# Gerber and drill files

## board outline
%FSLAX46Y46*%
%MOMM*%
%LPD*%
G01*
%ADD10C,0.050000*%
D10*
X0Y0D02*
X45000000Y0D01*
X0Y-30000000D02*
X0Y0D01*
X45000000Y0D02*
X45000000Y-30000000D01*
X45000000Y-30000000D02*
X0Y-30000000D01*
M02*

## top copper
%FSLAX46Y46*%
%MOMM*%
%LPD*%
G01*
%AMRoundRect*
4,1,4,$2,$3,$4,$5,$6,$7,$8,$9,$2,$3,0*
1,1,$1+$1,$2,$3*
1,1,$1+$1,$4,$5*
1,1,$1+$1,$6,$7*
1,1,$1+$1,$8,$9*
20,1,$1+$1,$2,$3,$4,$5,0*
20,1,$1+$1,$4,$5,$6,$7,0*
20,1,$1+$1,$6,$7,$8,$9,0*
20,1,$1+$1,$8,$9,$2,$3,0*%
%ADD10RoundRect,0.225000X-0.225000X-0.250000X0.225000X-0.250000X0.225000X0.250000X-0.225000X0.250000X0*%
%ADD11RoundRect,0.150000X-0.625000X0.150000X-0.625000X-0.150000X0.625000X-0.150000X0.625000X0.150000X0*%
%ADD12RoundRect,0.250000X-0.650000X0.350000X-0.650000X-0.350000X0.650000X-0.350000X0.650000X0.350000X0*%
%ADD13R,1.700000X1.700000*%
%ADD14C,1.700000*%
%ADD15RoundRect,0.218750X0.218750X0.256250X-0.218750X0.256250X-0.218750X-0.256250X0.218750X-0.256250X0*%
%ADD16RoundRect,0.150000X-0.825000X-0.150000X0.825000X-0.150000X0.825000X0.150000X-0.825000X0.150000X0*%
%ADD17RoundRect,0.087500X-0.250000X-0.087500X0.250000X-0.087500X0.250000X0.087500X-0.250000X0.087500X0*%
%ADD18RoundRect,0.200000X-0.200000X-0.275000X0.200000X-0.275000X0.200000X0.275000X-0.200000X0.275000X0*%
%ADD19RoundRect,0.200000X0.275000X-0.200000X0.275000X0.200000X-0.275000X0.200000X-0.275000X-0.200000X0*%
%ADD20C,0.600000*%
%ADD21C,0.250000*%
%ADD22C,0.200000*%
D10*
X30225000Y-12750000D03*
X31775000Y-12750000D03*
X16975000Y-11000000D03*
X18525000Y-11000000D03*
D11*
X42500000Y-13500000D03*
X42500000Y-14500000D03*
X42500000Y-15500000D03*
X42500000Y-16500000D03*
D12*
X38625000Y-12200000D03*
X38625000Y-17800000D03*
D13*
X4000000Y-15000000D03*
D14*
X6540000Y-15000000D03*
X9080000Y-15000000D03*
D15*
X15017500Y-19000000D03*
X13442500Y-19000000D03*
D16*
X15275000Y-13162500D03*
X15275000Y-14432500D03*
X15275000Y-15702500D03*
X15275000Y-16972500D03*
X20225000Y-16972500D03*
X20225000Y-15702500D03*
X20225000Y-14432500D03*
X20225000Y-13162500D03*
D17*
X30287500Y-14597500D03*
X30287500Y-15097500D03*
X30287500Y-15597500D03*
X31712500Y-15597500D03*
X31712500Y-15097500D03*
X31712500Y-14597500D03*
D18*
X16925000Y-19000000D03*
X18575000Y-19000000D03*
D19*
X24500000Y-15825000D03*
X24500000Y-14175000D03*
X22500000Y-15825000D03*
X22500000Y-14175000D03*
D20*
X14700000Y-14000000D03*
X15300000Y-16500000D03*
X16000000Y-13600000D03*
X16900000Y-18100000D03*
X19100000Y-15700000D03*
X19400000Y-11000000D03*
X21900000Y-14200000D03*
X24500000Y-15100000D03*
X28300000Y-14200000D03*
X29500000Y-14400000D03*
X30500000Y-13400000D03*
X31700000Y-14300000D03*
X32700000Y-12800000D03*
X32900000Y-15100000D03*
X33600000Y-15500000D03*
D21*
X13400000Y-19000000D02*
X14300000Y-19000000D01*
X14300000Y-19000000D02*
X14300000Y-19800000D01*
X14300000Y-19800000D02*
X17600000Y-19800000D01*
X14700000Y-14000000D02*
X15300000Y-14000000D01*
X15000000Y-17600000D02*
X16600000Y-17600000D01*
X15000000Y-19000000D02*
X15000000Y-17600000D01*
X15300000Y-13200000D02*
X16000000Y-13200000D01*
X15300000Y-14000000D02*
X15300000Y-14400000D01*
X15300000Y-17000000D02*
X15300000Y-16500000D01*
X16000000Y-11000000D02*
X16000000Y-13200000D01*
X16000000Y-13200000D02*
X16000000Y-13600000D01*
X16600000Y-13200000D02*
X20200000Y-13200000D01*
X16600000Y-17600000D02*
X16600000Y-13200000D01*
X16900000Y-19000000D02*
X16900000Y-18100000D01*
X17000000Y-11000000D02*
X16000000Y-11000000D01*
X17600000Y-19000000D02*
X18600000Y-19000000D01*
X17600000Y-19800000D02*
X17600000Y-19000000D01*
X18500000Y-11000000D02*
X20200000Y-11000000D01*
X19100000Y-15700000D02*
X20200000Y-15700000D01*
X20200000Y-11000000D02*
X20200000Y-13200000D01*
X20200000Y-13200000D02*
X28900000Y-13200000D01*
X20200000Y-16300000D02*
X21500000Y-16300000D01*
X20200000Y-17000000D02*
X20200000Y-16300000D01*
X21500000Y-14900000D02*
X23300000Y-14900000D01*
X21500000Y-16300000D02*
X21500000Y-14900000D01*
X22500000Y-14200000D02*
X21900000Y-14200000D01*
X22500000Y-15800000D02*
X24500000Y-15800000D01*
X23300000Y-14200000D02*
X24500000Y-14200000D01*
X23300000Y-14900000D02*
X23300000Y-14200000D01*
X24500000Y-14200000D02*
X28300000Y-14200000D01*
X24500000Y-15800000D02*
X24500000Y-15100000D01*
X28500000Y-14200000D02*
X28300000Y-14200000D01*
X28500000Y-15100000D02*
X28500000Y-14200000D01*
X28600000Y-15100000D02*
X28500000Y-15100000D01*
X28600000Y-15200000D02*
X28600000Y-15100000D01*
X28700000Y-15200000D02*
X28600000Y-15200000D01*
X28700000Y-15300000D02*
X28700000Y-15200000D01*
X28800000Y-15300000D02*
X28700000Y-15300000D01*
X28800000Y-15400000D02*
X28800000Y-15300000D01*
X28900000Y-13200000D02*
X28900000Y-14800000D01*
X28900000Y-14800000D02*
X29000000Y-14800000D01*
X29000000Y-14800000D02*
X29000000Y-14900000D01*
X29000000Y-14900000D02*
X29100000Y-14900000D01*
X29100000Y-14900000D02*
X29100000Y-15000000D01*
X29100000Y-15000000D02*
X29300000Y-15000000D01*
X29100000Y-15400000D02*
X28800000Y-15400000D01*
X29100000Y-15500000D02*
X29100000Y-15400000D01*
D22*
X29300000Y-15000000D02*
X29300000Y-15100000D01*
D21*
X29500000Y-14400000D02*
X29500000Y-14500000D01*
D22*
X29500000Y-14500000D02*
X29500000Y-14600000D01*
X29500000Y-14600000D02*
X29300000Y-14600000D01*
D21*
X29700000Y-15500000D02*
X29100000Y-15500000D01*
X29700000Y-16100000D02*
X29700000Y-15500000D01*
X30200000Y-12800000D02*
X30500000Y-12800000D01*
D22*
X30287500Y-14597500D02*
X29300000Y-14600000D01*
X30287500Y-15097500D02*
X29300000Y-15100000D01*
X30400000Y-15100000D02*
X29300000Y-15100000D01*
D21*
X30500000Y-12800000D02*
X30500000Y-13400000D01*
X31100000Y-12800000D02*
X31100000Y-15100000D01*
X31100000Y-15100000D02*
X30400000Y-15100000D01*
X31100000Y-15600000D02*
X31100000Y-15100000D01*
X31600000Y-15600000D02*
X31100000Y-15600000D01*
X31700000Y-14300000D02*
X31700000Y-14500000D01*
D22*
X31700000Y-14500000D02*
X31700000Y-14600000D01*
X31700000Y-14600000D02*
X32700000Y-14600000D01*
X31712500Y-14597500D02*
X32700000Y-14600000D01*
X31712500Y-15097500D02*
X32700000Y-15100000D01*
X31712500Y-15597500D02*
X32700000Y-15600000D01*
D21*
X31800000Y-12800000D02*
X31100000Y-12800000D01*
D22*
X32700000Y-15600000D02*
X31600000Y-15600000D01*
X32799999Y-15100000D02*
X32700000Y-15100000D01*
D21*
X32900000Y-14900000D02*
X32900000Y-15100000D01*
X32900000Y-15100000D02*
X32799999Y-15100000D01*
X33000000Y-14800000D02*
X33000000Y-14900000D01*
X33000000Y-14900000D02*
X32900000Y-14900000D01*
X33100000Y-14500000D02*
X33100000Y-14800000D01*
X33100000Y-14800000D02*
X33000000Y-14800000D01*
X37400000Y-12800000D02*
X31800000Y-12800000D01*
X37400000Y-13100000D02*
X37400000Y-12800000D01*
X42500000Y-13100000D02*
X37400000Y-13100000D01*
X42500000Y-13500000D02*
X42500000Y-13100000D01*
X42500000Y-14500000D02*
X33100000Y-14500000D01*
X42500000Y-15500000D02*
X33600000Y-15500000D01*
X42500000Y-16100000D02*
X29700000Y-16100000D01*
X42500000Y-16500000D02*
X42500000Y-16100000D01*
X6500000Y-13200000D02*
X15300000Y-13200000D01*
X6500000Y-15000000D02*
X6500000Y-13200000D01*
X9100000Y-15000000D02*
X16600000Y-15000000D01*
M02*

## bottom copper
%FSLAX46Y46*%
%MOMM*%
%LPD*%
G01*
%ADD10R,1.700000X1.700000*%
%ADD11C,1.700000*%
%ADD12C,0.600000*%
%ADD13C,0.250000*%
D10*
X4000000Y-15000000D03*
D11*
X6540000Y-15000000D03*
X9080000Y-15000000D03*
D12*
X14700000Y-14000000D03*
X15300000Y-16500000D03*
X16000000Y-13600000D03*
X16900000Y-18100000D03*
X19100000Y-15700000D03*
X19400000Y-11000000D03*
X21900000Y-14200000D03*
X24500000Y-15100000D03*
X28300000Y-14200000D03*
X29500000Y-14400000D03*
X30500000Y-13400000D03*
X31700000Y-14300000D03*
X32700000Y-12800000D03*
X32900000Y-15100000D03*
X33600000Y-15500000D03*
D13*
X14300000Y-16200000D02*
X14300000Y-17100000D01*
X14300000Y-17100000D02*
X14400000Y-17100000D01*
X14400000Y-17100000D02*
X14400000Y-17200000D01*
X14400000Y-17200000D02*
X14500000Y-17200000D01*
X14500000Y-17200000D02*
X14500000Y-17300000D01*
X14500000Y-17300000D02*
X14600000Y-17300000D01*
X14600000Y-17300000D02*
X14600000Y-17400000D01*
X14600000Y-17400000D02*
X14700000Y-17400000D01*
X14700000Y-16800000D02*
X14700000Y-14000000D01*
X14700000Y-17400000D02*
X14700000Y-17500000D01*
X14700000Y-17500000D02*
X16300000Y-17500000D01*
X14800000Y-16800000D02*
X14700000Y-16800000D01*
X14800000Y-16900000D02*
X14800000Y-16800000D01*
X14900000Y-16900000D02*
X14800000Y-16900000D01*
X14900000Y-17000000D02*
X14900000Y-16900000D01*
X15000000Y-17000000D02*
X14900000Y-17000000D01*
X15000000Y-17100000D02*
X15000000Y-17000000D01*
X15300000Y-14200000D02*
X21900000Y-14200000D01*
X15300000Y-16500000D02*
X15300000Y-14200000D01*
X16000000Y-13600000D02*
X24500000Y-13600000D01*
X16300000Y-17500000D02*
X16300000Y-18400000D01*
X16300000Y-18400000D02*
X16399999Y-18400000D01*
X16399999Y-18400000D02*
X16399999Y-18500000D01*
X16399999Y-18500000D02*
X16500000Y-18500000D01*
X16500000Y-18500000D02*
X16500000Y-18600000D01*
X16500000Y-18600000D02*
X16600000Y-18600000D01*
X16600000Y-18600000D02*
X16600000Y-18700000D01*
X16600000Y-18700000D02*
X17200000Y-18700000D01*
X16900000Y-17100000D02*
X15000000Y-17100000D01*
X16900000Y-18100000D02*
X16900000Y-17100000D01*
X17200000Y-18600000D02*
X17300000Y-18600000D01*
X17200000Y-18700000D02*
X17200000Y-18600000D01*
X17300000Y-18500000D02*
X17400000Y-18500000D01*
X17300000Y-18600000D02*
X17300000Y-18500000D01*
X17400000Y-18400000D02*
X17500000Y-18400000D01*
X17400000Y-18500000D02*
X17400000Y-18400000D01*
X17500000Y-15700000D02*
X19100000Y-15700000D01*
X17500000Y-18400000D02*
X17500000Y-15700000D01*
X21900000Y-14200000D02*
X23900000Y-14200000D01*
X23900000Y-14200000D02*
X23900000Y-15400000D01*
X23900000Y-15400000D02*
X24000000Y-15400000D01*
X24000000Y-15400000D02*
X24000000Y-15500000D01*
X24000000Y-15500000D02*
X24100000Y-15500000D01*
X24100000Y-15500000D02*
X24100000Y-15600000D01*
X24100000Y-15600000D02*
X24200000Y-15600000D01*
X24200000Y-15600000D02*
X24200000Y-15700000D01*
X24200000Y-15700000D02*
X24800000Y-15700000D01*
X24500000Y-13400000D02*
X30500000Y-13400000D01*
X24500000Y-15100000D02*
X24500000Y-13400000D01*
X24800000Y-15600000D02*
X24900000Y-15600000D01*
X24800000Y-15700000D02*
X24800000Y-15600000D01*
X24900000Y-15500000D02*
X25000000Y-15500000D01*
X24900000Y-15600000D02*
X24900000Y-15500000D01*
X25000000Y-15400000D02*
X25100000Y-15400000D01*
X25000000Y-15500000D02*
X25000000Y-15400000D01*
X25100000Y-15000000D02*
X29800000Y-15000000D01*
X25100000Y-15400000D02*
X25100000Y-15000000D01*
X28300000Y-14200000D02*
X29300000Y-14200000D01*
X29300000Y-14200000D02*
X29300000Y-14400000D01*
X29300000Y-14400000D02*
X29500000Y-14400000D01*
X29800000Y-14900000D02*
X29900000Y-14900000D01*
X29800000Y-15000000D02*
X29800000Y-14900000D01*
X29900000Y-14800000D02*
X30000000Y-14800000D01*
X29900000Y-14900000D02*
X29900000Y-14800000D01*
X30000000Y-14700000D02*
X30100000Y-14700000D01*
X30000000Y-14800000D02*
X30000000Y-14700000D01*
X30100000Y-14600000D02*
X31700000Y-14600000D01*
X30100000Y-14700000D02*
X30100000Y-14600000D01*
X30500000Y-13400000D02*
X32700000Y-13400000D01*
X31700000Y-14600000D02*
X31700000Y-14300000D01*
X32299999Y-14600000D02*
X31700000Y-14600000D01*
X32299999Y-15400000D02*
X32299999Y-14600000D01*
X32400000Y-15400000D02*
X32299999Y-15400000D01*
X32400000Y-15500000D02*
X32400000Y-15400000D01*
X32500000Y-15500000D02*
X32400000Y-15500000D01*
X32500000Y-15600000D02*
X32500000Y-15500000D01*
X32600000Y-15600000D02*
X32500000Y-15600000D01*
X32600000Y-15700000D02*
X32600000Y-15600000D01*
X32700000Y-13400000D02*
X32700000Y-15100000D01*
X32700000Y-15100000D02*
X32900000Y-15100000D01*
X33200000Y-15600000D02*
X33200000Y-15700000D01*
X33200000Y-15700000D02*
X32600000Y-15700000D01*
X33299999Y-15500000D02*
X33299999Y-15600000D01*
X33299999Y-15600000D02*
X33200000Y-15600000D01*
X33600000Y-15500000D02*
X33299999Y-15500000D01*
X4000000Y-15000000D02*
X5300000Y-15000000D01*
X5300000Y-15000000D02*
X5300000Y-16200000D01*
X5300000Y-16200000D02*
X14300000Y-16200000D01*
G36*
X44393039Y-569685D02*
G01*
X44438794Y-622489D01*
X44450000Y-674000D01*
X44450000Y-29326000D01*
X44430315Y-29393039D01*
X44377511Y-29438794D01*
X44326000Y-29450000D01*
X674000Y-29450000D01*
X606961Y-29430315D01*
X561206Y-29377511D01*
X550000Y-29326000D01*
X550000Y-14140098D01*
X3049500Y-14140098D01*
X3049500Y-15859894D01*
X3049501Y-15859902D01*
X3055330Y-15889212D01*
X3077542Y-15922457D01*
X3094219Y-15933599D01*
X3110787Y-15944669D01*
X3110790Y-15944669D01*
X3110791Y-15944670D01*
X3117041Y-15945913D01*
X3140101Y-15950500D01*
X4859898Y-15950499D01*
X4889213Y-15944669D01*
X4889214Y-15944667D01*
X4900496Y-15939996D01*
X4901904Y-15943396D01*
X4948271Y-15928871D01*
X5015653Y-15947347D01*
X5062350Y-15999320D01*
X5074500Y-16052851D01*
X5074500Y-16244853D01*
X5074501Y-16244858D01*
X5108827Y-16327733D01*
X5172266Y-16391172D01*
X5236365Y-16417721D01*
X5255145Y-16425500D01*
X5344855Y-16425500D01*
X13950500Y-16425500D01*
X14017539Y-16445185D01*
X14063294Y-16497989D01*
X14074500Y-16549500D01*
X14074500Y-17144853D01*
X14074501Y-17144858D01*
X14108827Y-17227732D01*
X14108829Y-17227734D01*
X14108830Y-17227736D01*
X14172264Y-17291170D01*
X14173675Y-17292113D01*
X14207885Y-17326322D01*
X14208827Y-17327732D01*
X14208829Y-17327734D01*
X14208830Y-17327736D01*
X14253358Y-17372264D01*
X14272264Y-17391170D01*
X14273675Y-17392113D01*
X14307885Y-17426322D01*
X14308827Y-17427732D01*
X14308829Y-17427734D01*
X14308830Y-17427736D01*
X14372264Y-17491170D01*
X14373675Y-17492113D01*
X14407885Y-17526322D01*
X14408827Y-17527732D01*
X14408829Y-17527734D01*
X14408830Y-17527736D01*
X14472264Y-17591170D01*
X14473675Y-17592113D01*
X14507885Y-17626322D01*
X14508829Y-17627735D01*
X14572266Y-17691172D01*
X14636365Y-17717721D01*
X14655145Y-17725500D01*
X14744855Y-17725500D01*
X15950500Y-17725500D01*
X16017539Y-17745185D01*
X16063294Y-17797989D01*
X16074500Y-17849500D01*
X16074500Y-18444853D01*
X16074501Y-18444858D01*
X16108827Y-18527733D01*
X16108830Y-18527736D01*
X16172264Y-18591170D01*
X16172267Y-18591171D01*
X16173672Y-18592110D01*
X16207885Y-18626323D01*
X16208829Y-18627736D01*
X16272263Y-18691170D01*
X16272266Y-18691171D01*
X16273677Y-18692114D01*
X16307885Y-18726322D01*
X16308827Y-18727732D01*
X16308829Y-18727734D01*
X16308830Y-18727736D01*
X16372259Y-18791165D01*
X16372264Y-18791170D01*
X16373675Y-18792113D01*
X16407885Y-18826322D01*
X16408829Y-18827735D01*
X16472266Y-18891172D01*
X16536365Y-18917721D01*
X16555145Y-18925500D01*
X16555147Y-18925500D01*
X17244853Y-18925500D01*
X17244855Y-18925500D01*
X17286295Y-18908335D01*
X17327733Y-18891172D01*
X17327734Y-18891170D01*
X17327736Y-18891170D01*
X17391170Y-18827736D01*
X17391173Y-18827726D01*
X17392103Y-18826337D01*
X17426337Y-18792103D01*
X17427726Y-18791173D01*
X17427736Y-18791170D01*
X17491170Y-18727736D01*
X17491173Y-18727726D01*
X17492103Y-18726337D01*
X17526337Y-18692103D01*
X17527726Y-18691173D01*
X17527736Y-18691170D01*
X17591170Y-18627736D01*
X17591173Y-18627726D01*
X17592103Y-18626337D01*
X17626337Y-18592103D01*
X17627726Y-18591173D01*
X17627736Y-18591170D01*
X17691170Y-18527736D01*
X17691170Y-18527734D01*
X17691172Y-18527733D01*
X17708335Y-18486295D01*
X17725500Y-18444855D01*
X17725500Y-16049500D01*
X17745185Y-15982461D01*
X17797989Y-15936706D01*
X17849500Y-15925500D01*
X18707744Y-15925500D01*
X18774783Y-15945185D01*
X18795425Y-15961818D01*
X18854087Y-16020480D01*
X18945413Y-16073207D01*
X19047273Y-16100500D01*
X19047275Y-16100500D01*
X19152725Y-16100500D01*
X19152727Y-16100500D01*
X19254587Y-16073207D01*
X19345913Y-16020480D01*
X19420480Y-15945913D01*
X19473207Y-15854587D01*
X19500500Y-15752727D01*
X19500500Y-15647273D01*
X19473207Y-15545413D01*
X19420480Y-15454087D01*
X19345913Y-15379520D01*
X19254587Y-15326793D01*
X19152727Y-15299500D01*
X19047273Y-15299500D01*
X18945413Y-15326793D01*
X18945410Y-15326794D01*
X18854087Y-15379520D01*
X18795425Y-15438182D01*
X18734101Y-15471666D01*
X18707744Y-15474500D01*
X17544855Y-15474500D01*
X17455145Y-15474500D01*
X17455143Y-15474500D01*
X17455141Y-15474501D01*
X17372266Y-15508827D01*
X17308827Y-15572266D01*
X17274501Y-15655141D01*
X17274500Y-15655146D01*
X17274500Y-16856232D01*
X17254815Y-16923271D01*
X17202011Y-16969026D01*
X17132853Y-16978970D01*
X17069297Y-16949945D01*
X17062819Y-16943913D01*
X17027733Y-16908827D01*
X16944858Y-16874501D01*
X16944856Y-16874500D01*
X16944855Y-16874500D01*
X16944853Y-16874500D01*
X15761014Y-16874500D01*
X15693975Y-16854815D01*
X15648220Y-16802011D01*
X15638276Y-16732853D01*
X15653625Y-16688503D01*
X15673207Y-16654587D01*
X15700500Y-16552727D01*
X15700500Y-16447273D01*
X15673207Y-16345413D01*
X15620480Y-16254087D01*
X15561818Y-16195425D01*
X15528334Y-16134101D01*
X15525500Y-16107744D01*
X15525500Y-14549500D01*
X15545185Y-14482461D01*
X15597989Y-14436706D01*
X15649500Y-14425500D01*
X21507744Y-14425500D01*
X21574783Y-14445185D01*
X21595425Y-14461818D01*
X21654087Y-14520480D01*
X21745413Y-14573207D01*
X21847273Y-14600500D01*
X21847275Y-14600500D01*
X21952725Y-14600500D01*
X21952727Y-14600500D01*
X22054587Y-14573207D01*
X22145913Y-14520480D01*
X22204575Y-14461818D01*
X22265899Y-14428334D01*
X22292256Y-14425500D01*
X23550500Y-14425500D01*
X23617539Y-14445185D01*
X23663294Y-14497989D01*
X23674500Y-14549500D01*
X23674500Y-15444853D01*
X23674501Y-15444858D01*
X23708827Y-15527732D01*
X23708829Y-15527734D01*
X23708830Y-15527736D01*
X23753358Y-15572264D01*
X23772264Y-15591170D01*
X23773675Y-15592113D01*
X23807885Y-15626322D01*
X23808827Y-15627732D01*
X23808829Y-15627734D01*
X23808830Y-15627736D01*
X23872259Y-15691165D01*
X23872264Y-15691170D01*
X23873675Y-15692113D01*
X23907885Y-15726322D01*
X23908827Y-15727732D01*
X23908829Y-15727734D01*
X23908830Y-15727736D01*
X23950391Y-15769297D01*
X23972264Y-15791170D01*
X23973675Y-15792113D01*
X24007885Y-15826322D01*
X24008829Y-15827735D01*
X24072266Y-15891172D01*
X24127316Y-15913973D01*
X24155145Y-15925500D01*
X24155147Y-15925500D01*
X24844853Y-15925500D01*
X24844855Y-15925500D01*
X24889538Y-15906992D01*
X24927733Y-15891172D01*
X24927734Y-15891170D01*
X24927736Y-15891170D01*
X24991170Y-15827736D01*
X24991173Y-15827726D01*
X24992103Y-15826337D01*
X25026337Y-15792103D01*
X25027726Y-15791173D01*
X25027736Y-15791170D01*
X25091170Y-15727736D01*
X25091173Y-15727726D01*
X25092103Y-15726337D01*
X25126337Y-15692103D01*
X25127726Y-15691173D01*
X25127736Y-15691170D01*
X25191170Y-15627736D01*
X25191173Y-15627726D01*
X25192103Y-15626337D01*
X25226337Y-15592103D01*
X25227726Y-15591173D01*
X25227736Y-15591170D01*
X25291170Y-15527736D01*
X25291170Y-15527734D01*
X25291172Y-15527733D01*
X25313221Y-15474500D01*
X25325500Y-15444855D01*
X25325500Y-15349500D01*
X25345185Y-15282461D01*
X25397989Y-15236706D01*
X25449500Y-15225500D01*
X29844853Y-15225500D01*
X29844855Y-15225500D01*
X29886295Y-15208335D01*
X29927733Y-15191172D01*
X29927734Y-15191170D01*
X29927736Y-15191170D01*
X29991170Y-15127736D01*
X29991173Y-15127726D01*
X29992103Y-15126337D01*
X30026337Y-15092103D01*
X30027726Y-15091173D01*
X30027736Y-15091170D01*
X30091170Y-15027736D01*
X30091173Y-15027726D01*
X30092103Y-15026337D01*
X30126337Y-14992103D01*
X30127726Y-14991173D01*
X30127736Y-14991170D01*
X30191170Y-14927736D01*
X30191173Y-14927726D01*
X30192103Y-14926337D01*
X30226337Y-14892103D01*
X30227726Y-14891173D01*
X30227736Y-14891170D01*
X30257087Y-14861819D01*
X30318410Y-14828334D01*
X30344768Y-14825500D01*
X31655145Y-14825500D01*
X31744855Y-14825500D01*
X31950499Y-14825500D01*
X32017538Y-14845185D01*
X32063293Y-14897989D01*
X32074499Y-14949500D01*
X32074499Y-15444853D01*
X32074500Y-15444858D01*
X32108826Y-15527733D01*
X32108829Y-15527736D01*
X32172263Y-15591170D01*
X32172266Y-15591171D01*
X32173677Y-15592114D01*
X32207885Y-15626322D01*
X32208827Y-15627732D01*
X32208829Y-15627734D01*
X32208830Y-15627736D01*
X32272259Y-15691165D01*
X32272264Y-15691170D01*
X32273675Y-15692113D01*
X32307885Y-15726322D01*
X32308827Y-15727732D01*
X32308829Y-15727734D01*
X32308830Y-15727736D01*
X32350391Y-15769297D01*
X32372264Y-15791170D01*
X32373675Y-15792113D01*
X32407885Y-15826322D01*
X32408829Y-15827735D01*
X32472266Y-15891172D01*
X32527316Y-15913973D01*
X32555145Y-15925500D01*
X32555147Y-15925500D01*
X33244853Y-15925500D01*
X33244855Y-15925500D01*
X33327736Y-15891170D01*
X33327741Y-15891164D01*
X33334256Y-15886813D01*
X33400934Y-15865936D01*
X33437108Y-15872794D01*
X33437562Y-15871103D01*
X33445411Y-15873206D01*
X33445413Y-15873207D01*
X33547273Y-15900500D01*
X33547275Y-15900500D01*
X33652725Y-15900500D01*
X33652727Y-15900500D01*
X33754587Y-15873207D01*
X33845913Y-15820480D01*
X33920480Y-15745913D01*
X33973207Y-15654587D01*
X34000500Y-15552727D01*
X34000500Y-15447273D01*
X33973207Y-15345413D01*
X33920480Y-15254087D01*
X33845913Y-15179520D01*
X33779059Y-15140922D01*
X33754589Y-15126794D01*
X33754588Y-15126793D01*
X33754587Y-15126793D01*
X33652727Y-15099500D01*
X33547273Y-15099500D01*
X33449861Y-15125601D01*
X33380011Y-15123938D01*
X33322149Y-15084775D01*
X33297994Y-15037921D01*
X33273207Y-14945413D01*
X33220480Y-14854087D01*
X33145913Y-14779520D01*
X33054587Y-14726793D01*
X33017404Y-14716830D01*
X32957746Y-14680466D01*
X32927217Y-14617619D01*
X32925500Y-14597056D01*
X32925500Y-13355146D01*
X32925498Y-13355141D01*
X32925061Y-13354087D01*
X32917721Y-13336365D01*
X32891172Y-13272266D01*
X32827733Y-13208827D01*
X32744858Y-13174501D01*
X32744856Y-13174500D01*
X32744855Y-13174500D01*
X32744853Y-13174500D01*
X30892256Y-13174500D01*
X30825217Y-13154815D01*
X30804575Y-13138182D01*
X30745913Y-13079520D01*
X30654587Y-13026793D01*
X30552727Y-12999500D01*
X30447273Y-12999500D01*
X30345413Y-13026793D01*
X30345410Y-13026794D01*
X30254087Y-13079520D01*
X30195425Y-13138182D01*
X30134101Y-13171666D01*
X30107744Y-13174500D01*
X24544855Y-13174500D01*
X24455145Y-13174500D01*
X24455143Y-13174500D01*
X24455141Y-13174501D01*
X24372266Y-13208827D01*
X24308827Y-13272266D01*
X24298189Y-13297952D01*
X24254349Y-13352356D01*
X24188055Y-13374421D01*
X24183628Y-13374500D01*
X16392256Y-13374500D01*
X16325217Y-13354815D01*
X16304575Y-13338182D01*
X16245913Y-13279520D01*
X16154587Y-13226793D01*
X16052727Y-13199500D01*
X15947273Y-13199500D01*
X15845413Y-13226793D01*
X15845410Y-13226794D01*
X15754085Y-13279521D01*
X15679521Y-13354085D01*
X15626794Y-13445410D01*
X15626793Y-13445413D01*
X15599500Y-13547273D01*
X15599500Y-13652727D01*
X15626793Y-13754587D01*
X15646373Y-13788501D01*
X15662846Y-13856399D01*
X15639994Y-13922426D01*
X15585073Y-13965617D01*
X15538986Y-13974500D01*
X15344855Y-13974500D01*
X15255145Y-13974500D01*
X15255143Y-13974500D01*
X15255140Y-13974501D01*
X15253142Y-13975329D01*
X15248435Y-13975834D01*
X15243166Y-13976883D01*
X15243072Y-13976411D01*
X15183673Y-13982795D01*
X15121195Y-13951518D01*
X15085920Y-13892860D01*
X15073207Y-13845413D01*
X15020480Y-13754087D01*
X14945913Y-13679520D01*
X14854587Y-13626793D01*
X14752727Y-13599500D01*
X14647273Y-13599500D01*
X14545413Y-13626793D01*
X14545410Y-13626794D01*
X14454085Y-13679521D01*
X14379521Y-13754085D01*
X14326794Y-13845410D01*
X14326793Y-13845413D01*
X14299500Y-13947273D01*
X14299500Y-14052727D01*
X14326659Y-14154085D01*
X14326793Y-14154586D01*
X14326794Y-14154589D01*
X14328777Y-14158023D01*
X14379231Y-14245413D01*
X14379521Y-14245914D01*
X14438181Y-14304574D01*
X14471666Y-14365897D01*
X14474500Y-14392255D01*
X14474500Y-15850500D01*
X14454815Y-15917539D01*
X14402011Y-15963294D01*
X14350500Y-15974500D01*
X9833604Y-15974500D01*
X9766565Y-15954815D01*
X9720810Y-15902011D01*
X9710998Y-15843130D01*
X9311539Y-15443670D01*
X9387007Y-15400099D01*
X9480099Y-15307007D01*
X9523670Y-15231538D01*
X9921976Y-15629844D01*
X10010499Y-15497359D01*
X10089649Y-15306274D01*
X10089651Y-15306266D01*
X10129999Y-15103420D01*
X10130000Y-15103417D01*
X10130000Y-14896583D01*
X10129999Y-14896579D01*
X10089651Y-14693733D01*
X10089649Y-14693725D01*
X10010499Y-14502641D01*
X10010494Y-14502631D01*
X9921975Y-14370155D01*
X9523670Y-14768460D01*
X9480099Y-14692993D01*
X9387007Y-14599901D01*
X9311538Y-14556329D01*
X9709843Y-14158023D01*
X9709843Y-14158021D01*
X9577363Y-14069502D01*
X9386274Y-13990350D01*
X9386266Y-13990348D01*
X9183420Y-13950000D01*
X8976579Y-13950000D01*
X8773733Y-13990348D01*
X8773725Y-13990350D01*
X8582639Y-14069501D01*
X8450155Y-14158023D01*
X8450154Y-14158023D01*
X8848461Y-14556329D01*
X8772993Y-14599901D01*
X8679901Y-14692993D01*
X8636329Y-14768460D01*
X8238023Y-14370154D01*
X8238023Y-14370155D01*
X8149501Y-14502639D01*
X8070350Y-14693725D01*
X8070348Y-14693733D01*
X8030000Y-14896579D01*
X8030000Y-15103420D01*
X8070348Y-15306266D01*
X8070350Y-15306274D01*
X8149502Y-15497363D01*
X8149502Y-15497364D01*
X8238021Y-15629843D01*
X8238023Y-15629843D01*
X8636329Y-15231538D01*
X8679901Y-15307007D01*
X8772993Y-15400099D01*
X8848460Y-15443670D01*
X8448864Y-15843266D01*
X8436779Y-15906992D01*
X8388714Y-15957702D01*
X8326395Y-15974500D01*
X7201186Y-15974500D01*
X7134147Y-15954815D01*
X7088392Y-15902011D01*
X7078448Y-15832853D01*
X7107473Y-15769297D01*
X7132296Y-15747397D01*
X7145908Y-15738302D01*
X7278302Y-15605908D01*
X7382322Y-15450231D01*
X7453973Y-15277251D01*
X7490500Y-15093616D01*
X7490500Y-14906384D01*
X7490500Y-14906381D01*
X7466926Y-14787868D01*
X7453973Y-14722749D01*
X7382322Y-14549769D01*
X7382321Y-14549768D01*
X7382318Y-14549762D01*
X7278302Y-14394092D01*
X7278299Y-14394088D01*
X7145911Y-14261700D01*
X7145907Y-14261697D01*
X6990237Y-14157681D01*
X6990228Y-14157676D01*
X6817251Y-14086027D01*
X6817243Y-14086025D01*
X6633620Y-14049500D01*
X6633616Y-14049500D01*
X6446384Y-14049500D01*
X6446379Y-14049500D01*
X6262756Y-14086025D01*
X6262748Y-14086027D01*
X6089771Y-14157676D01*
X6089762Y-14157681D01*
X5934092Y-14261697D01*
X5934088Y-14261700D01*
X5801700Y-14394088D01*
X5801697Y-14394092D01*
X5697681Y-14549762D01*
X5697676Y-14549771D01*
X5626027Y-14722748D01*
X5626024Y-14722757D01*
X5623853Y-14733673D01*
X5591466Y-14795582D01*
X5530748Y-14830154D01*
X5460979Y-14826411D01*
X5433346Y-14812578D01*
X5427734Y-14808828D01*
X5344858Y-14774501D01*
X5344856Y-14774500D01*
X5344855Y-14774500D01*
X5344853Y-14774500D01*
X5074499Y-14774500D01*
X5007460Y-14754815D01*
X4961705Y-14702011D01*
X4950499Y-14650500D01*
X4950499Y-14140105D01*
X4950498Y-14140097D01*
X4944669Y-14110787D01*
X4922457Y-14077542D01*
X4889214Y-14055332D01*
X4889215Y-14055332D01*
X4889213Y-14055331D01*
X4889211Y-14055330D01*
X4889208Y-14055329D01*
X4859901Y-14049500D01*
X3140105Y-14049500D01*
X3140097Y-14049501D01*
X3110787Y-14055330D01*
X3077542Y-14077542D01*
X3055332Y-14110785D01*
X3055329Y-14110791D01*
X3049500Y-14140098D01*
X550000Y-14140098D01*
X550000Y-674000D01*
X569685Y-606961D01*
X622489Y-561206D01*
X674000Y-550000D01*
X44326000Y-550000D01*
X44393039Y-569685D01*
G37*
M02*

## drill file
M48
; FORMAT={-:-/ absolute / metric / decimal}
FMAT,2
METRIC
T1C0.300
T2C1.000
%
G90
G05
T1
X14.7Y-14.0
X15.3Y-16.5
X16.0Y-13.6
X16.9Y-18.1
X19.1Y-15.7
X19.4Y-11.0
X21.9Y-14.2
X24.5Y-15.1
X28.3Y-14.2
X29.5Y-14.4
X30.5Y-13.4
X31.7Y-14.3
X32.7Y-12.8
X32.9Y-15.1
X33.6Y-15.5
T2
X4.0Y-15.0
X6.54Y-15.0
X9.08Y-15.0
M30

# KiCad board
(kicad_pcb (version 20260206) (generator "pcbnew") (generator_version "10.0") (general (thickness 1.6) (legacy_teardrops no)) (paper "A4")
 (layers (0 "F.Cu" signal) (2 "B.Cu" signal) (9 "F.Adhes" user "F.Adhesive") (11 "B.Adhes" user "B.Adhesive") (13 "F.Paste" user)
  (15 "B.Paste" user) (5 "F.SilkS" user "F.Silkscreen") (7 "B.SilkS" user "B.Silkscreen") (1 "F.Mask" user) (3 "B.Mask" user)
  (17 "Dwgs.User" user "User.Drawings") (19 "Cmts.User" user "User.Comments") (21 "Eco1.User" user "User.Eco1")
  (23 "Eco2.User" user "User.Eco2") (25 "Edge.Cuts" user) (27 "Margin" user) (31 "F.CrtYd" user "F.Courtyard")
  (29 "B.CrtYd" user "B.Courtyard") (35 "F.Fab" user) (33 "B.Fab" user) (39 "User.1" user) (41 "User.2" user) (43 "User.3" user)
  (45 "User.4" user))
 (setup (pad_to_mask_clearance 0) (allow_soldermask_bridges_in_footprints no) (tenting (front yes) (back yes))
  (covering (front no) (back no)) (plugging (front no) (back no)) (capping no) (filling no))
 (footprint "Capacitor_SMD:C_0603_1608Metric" (layer "F.Cu") (at 31 12.75)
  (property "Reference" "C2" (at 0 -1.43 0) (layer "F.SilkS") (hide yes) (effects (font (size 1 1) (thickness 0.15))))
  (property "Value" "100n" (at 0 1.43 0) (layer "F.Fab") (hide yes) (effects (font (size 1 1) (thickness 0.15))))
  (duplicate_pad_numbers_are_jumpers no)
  (pad "1" smd roundrect (at -0.775 0) (size 0.9 0.95) (layers "F.Cu" "F.Mask" "F.Paste") (roundrect_rratio 0.25) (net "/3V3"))
  (pad "2" smd roundrect (at 0.775 0) (size 0.9 0.95) (layers "F.Cu" "F.Mask" "F.Paste") (roundrect_rratio 0.25) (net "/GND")))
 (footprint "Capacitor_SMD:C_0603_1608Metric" (layer "F.Cu") (at 17.75 11)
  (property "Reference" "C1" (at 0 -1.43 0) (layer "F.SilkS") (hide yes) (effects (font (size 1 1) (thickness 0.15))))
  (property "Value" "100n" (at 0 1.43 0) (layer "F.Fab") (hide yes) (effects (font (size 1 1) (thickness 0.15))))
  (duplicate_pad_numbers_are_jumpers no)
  (pad "1" smd roundrect (at -0.775 0) (size 0.9 0.95) (layers "F.Cu" "F.Mask" "F.Paste") (roundrect_rratio 0.25) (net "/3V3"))
  (pad "2" smd roundrect (at 0.775 0) (size 0.9 0.95) (layers "F.Cu" "F.Mask" "F.Paste") (roundrect_rratio 0.25) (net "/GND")))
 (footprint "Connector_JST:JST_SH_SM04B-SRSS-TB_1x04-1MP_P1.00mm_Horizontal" (layer "F.Cu") (at 40.5 15 -90)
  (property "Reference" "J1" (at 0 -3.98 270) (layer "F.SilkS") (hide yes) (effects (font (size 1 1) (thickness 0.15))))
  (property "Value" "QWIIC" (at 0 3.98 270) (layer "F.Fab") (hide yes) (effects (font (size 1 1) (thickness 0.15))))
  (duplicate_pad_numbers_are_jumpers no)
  (pad "1" smd roundrect (at -1.5 -2 270) (size 0.6 1.55) (layers "F.Cu" "F.Mask" "F.Paste") (roundrect_rratio 0.25) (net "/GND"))
  (pad "2" smd roundrect (at -0.5 -2 270) (size 0.6 1.55) (layers "F.Cu" "F.Mask" "F.Paste") (roundrect_rratio 0.25) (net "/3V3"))
  (pad "3" smd roundrect (at 0.5 -2 270) (size 0.6 1.55) (layers "F.Cu" "F.Mask" "F.Paste") (roundrect_rratio 0.25) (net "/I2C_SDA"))
  (pad "4" smd roundrect (at 1.5 -2 270) (size 0.6 1.55) (layers "F.Cu" "F.Mask" "F.Paste") (roundrect_rratio 0.25) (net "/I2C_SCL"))
  (pad "MP" smd roundrect (at -2.8 1.875 270) (size 1.2 1.8) (layers "F.Cu" "F.Mask" "F.Paste") (roundrect_rratio 0.208333))
  (pad "MP" smd roundrect (at 2.8 1.875 270) (size 1.2 1.8) (layers "F.Cu" "F.Mask" "F.Paste") (roundrect_rratio 0.208333)))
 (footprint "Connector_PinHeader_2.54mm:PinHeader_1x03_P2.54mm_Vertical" (layer "F.Cu") (at 4 15 90)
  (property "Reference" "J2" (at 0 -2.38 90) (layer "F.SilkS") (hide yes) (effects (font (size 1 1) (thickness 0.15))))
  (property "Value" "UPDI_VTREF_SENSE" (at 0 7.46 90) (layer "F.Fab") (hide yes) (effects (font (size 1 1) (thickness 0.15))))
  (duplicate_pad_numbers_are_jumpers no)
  (pad "1" thru_hole rect (at 0 0 90) (size 1.7 1.7) (drill 1) (layers "*.Cu" "*.Mask") (remove_unused_layers no) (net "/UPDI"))
  (pad "2" thru_hole circle (at 0 2.54 90) (size 1.7 1.7) (drill 1) (layers "*.Cu" "*.Mask") (remove_unused_layers no) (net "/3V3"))
  (pad "3" thru_hole circle (at 0 5.08 90) (size 1.7 1.7) (drill 1) (layers "*.Cu" "*.Mask") (remove_unused_layers no) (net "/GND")))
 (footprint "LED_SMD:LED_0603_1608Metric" (layer "F.Cu") (at 14.23 19 180)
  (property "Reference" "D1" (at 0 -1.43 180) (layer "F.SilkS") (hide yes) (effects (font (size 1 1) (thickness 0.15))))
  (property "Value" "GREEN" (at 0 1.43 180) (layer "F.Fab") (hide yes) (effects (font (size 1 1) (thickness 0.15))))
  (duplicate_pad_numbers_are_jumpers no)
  (pad "1" smd roundrect (at -0.7875 0 180) (size 0.875 0.95) (layers "F.Cu" "F.Mask" "F.Paste") (roundrect_rratio 0.25) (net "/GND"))
  (pad "2" smd roundrect (at 0.7875 0 180) (size 0.875 0.95) (layers "F.Cu" "F.Mask" "F.Paste") (roundrect_rratio 0.25) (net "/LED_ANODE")))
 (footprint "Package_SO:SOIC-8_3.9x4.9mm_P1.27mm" (layer "F.Cu") (at 17.75 15.0675)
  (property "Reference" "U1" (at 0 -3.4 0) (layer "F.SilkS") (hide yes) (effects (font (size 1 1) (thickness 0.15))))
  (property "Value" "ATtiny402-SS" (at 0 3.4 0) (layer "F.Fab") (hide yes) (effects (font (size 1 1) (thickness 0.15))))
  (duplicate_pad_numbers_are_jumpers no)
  (pad "1" smd roundrect (at -2.475 -1.905) (size 1.95 0.6) (layers "F.Cu" "F.Mask" "F.Paste") (roundrect_rratio 0.25) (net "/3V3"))
  (pad "2" smd roundrect (at -2.475 -0.635) (size 1.95 0.6) (layers "F.Cu" "F.Mask" "F.Paste") (roundrect_rratio 0.25) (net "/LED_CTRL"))
  (pad "3" smd roundrect (at -2.475 0.635) (size 1.95 0.6) (layers "F.Cu" "F.Mask" "F.Paste") (roundrect_rratio 0.25)
   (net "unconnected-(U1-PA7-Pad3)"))
  (pad "4" smd roundrect (at -2.475 1.905) (size 1.95 0.6) (layers "F.Cu" "F.Mask" "F.Paste") (roundrect_rratio 0.25) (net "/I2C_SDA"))
  (pad "5" smd roundrect (at 2.475 1.905) (size 1.95 0.6) (layers "F.Cu" "F.Mask" "F.Paste") (roundrect_rratio 0.25) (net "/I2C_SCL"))
  (pad "6" smd roundrect (at 2.475 0.635) (size 1.95 0.6) (layers "F.Cu" "F.Mask" "F.Paste") (roundrect_rratio 0.25) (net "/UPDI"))
  (pad "7" smd roundrect (at 2.475 -0.635) (size 1.95 0.6) (layers "F.Cu" "F.Mask" "F.Paste") (roundrect_rratio 0.25)
   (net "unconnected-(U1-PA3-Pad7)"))
  (pad "8" smd roundrect (at 2.475 -1.905) (size 1.95 0.6) (layers "F.Cu" "F.Mask" "F.Paste") (roundrect_rratio 0.25) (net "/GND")))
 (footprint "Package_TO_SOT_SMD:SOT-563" (layer "F.Cu") (at 31 15.0975)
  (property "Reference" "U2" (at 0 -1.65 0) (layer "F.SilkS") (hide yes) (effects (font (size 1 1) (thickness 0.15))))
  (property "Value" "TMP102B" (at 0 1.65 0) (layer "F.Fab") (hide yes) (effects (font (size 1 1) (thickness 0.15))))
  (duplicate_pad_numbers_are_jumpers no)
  (pad "1" smd roundrect (at -0.7125 -0.5) (size 0.675 0.35) (layers "F.Cu" "F.Mask" "F.Paste") (roundrect_rratio 0.25) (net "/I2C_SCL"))
  (pad "2" smd roundrect (at -0.7125 0) (size 0.675 0.35) (layers "F.Cu" "F.Mask" "F.Paste") (roundrect_rratio 0.25) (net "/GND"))
  (pad "3" smd roundrect (at -0.7125 0.5) (size 0.675 0.35) (layers "F.Cu" "F.Mask" "F.Paste") (roundrect_rratio 0.25)
   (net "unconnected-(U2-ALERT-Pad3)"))
  (pad "4" smd roundrect (at 0.7125 0.5) (size 0.675 0.35) (layers "F.Cu" "F.Mask" "F.Paste") (roundrect_rratio 0.25) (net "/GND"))
  (pad "5" smd roundrect (at 0.7125 0) (size 0.675 0.35) (layers "F.Cu" "F.Mask" "F.Paste") (roundrect_rratio 0.25) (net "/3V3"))
  (pad "6" smd roundrect (at 0.7125 -0.5) (size 0.675 0.35) (layers "F.Cu" "F.Mask" "F.Paste") (roundrect_rratio 0.25) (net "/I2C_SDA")))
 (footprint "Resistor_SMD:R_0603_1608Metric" (layer "F.Cu") (at 17.75 19)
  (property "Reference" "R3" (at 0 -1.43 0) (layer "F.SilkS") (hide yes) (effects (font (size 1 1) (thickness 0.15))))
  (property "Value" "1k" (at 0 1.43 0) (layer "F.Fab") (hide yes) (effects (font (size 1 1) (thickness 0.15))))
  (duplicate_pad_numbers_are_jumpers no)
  (pad "1" smd roundrect (at -0.825 0) (size 0.8 0.95) (layers "F.Cu" "F.Mask" "F.Paste") (roundrect_rratio 0.25) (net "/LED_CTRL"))
  (pad "2" smd roundrect (at 0.825 0) (size 0.8 0.95) (layers "F.Cu" "F.Mask" "F.Paste") (roundrect_rratio 0.25) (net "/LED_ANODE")))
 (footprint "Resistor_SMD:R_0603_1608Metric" (layer "F.Cu") (at 24.5 15 90)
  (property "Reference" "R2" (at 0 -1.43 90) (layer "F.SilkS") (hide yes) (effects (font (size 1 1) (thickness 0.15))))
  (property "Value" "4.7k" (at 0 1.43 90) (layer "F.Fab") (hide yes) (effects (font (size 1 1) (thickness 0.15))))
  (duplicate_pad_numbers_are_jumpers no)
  (pad "1" smd roundrect (at -0.825 0 90) (size 0.8 0.95) (layers "F.Cu" "F.Mask" "F.Paste") (roundrect_rratio 0.25) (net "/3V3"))
  (pad "2" smd roundrect (at 0.825 0 90) (size 0.8 0.95) (layers "F.Cu" "F.Mask" "F.Paste") (roundrect_rratio 0.25) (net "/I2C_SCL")))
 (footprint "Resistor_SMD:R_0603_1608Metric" (layer "F.Cu") (at 22.5 15 90)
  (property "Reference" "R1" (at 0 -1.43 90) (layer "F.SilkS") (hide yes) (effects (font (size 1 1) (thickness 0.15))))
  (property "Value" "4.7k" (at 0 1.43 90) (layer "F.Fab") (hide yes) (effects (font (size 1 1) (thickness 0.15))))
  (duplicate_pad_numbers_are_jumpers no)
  (pad "1" smd roundrect (at -0.825 0 90) (size 0.8 0.95) (layers "F.Cu" "F.Mask" "F.Paste") (roundrect_rratio 0.25) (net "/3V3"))
  (pad "2" smd roundrect (at 0.825 0 90) (size 0.8 0.95) (layers "F.Cu" "F.Mask" "F.Paste") (roundrect_rratio 0.25) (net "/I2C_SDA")))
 (gr_line (start 0 0) (end 45 0) (stroke (width 0.05) (type default)) (layer "Edge.Cuts"))
 (gr_line (start 0 30) (end 0 0) (stroke (width 0.05) (type default)) (layer "Edge.Cuts"))
 (gr_line (start 45 0) (end 45 30) (stroke (width 0.05) (type default)) (layer "Edge.Cuts"))
 (gr_line (start 45 30) (end 0 30) (stroke (width 0.05) (type default)) (layer "Edge.Cuts"))
 (segment (start 13.4 19) (end 14.3 19) (width 0.25) (layer "F.Cu") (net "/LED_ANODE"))
 (segment (start 14.3 16.2) (end 14.3 17.1) (width 0.25) (layer "B.Cu") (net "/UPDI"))
 (segment (start 14.3 17.1) (end 14.4 17.1) (width 0.25) (layer "B.Cu") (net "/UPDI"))
 (segment (start 14.3 19) (end 14.3 19.8) (width 0.25) (layer "F.Cu") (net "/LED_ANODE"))
 (segment (start 14.3 19.8) (end 17.6 19.8) (width 0.25) (layer "F.Cu") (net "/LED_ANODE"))
 (segment (start 14.4 17.1) (end 14.4 17.2) (width 0.25) (layer "B.Cu") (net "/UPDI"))
 (segment (start 14.4 17.2) (end 14.5 17.2) (width 0.25) (layer "B.Cu") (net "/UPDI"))
 (segment (start 14.5 17.2) (end 14.5 17.3) (width 0.25) (layer "B.Cu") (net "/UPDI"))
 (segment (start 14.5 17.3) (end 14.6 17.3) (width 0.25) (layer "B.Cu") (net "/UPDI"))
 (segment (start 14.6 17.3) (end 14.6 17.4) (width 0.25) (layer "B.Cu") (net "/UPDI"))
 (segment (start 14.6 17.4) (end 14.7 17.4) (width 0.25) (layer "B.Cu") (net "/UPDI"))
 (segment (start 14.7 14) (end 15.3 14) (width 0.25) (layer "F.Cu") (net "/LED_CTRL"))
 (segment (start 14.7 16.8) (end 14.7 14) (width 0.25) (layer "B.Cu") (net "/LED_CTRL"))
 (segment (start 14.7 17.4) (end 14.7 17.5) (width 0.25) (layer "B.Cu") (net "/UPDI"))
 (segment (start 14.7 17.5) (end 16.3 17.5) (width 0.25) (layer "B.Cu") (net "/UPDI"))
 (segment (start 14.8 16.8) (end 14.7 16.8) (width 0.25) (layer "B.Cu") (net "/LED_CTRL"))
 (segment (start 14.8 16.9) (end 14.8 16.8) (width 0.25) (layer "B.Cu") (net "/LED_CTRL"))
 (segment (start 14.9 16.9) (end 14.8 16.9) (width 0.25) (layer "B.Cu") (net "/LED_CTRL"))
 (segment (start 14.9 17) (end 14.9 16.9) (width 0.25) (layer "B.Cu") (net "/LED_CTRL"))
 (segment (start 15 17) (end 14.9 17) (width 0.25) (layer "B.Cu") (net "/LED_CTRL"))
 (segment (start 15 17.1) (end 15 17) (width 0.25) (layer "B.Cu") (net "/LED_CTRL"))
 (segment (start 15 17.6) (end 16.6 17.6) (width 0.25) (layer "F.Cu") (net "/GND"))
 (segment (start 15 19) (end 15 17.6) (width 0.25) (layer "F.Cu") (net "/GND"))
 (segment (start 15.3 13.2) (end 16 13.2) (width 0.25) (layer "F.Cu") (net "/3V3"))
 (segment (start 15.3 14) (end 15.3 14.4) (width 0.25) (layer "F.Cu") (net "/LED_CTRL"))
 (segment (start 15.3 14.2) (end 21.9 14.2) (width 0.25) (layer "B.Cu") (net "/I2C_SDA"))
 (segment (start 15.3 16.5) (end 15.3 14.2) (width 0.25) (layer "B.Cu") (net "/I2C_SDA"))
 (segment (start 15.3 17) (end 15.3 16.5) (width 0.25) (layer "F.Cu") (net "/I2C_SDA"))
 (segment (start 16 11) (end 16 13.2) (width 0.25) (layer "F.Cu") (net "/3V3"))
 (segment (start 16 13.2) (end 16 13.6) (width 0.25) (layer "F.Cu") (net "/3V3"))
 (segment (start 16 13.6) (end 24.5 13.6) (width 0.25) (layer "B.Cu") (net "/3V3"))
 (segment (start 16.3 17.5) (end 16.3 18.4) (width 0.25) (layer "B.Cu") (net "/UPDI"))
 (segment (start 16.3 18.4) (end 16.399999 18.4) (width 0.25) (layer "B.Cu") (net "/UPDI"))
 (segment (start 16.399999 18.4) (end 16.399999 18.5) (width 0.25) (layer "B.Cu") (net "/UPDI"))
 (segment (start 16.399999 18.5) (end 16.5 18.5) (width 0.25) (layer "B.Cu") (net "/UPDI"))
 (segment (start 16.5 18.5) (end 16.5 18.6) (width 0.25) (layer "B.Cu") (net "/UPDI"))
 (segment (start 16.5 18.6) (end 16.6 18.6) (width 0.25) (layer "B.Cu") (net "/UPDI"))
 (segment (start 16.6 13.2) (end 20.2 13.2) (width 0.25) (layer "F.Cu") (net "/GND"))
 (segment (start 16.6 17.6) (end 16.6 13.2) (width 0.25) (layer "F.Cu") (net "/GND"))
 (segment (start 16.6 18.6) (end 16.6 18.7) (width 0.25) (layer "B.Cu") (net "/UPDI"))
 (segment (start 16.6 18.7) (end 17.2 18.7) (width 0.25) (layer "B.Cu") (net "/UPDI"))
 (segment (start 16.9 17.1) (end 15 17.1) (width 0.25) (layer "B.Cu") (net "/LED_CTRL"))
 (segment (start 16.9 18.1) (end 16.9 17.1) (width 0.25) (layer "B.Cu") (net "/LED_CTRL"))
 (segment (start 16.9 19) (end 16.9 18.1) (width 0.25) (layer "F.Cu") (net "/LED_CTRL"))
 (segment (start 17 11) (end 16 11) (width 0.25) (layer "F.Cu") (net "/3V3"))
 (segment (start 17.2 18.6) (end 17.3 18.6) (width 0.25) (layer "B.Cu") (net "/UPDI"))
 (segment (start 17.2 18.7) (end 17.2 18.6) (width 0.25) (layer "B.Cu") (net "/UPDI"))
 (segment (start 17.3 18.5) (end 17.4 18.5) (width 0.25) (layer "B.Cu") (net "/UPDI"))
 (segment (start 17.3 18.6) (end 17.3 18.5) (width 0.25) (layer "B.Cu") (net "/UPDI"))
 (segment (start 17.4 18.4) (end 17.5 18.4) (width 0.25) (layer "B.Cu") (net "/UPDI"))
 (segment (start 17.4 18.5) (end 17.4 18.4) (width 0.25) (layer "B.Cu") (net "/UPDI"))
 (segment (start 17.5 15.7) (end 19.1 15.7) (width 0.25) (layer "B.Cu") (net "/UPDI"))
 (segment (start 17.5 18.4) (end 17.5 15.7) (width 0.25) (layer "B.Cu") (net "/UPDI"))
 (segment (start 17.6 19) (end 18.6 19) (width 0.25) (layer "F.Cu") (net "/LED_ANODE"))
 (segment (start 17.6 19.8) (end 17.6 19) (width 0.25) (layer "F.Cu") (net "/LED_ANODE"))
 (segment (start 18.5 11) (end 20.2 11) (width 0.25) (layer "F.Cu") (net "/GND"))
 (segment (start 19.1 15.7) (end 20.2 15.7) (width 0.25) (layer "F.Cu") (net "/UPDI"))
 (segment (start 20.2 11) (end 20.2 13.2) (width 0.25) (layer "F.Cu") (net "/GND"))
 (segment (start 20.2 13.2) (end 28.9 13.2) (width 0.25) (layer "F.Cu") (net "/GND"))
 (segment (start 20.2 16.3) (end 21.5 16.3) (width 0.25) (layer "F.Cu") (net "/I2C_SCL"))
 (segment (start 20.2 17) (end 20.2 16.3) (width 0.25) (layer "F.Cu") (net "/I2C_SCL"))
 (segment (start 21.5 14.9) (end 23.3 14.9) (width 0.25) (layer "F.Cu") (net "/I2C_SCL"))
 (segment (start 21.5 16.3) (end 21.5 14.9) (width 0.25) (layer "F.Cu") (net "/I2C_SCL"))
 (segment (start 21.9 14.2) (end 23.9 14.2) (width 0.25) (layer "B.Cu") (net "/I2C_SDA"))
 (segment (start 22.5 14.2) (end 21.9 14.2) (width 0.25) (layer "F.Cu") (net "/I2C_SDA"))
 (segment (start 22.5 15.8) (end 24.5 15.8) (width 0.25) (layer "F.Cu") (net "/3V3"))
 (segment (start 23.3 14.2) (end 24.5 14.2) (width 0.25) (layer "F.Cu") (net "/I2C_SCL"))
 (segment (start 23.3 14.9) (end 23.3 14.2) (width 0.25) (layer "F.Cu") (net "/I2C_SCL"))
 (segment (start 23.9 14.2) (end 23.9 15.4) (width 0.25) (layer "B.Cu") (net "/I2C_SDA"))
 (segment (start 23.9 15.4) (end 24 15.4) (width 0.25) (layer "B.Cu") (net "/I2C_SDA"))
 (segment (start 24 15.4) (end 24 15.5) (width 0.25) (layer "B.Cu") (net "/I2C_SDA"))
 (segment (start 24 15.5) (end 24.1 15.5) (width 0.25) (layer "B.Cu") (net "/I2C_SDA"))
 (segment (start 24.1 15.5) (end 24.1 15.6) (width 0.25) (layer "B.Cu") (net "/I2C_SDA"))
 (segment (start 24.1 15.6) (end 24.2 15.6) (width 0.25) (layer "B.Cu") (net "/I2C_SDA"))
 (segment (start 24.2 15.6) (end 24.2 15.7) (width 0.25) (layer "B.Cu") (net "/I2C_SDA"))
 (segment (start 24.2 15.7) (end 24.8 15.7) (width 0.25) (layer "B.Cu") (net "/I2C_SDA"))
 (segment (start 24.5 13.4) (end 30.5 13.4) (width 0.25) (layer "B.Cu") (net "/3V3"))
 (segment (start 24.5 14.2) (end 28.3 14.2) (width 0.25) (layer "F.Cu") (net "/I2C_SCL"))
 (segment (start 24.5 15.1) (end 24.5 13.4) (width 0.25) (layer "B.Cu") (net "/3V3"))
 (segment (start 24.5 15.8) (end 24.5 15.1) (width 0.25) (layer "F.Cu") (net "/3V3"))
 (segment (start 24.8 15.6) (end 24.9 15.6) (width 0.25) (layer "B.Cu") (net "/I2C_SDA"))
 (segment (start 24.8 15.7) (end 24.8 15.6) (width 0.25) (layer "B.Cu") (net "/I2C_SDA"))
 (segment (start 24.9 15.5) (end 25 15.5) (width 0.25) (layer "B.Cu") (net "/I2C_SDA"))
 (segment (start 24.9 15.6) (end 24.9 15.5) (width 0.25) (layer "B.Cu") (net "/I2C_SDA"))
 (segment (start 25 15.4) (end 25.1 15.4) (width 0.25) (layer "B.Cu") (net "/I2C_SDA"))
 (segment (start 25 15.5) (end 25 15.4) (width 0.25) (layer "B.Cu") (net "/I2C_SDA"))
 (segment (start 25.1 15) (end 29.8 15) (width 0.25) (layer "B.Cu") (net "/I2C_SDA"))
 (segment (start 25.1 15.4) (end 25.1 15) (width 0.25) (layer "B.Cu") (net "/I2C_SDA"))
 (segment (start 28.3 14.2) (end 29.3 14.2) (width 0.25) (layer "B.Cu") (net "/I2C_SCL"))
 (segment (start 28.5 14.2) (end 28.3 14.2) (width 0.25) (layer "F.Cu") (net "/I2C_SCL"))
 (segment (start 28.5 15.1) (end 28.5 14.2) (width 0.25) (layer "F.Cu") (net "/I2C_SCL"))
 (segment (start 28.6 15.1) (end 28.5 15.1) (width 0.25) (layer "F.Cu") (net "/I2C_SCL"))
 (segment (start 28.6 15.2) (end 28.6 15.1) (width 0.25) (layer "F.Cu") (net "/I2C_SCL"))
 (segment (start 28.7 15.2) (end 28.6 15.2) (width 0.25) (layer "F.Cu") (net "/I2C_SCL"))
 (segment (start 28.7 15.3) (end 28.7 15.2) (width 0.25) (layer "F.Cu") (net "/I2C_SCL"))
 (segment (start 28.8 15.3) (end 28.7 15.3) (width 0.25) (layer "F.Cu") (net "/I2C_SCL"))
 (segment (start 28.8 15.4) (end 28.8 15.3) (width 0.25) (layer "F.Cu") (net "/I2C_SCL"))
 (segment (start 28.9 13.2) (end 28.9 14.8) (width 0.25) (layer "F.Cu") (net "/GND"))
 (segment (start 28.9 14.8) (end 29 14.8) (width 0.25) (layer "F.Cu") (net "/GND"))
 (segment (start 29 14.8) (end 29 14.9) (width 0.25) (layer "F.Cu") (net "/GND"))
 (segment (start 29 14.9) (end 29.1 14.9) (width 0.25) (layer "F.Cu") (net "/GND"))
 (segment (start 29.1 14.9) (end 29.1 15) (width 0.25) (layer "F.Cu") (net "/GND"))
 (segment (start 29.1 15) (end 29.3 15) (width 0.25) (layer "F.Cu") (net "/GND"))
 (segment (start 29.1 15.4) (end 28.8 15.4) (width 0.25) (layer "F.Cu") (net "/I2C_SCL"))
 (segment (start 29.1 15.5) (end 29.1 15.4) (width 0.25) (layer "F.Cu") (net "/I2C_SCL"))
 (segment (start 29.3 14.2) (end 29.3 14.4) (width 0.25) (layer "B.Cu") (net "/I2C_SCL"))
 (segment (start 29.3 14.4) (end 29.5 14.4) (width 0.25) (layer "B.Cu") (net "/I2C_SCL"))
 (segment (start 29.3 15) (end 29.3 15.1) (width 0.2) (layer "F.Cu") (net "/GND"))
 (segment (start 29.5 14.4) (end 29.5 14.5) (width 0.25) (layer "F.Cu") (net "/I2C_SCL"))
 (segment (start 29.5 14.5) (end 29.5 14.6) (width 0.2) (layer "F.Cu") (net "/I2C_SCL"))
 (segment (start 29.5 14.6) (end 29.3 14.6) (width 0.2) (layer "F.Cu") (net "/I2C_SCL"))
 (segment (start 29.7 15.5) (end 29.1 15.5) (width 0.25) (layer "F.Cu") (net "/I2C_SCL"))
 (segment (start 29.7 16.1) (end 29.7 15.5) (width 0.25) (layer "F.Cu") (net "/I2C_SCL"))
 (segment (start 29.8 14.9) (end 29.9 14.9) (width 0.25) (layer "B.Cu") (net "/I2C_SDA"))
 (segment (start 29.8 15) (end 29.8 14.9) (width 0.25) (layer "B.Cu") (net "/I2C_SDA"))
 (segment (start 29.9 14.8) (end 30 14.8) (width 0.25) (layer "B.Cu") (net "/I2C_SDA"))
 (segment (start 29.9 14.9) (end 29.9 14.8) (width 0.25) (layer "B.Cu") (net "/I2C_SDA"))
 (segment (start 30 14.7) (end 30.1 14.7) (width 0.25) (layer "B.Cu") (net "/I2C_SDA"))
 (segment (start 30 14.8) (end 30 14.7) (width 0.25) (layer "B.Cu") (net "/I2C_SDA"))
 (segment (start 30.1 14.6) (end 31.7 14.6) (width 0.25) (layer "B.Cu") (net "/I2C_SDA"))
 (segment (start 30.1 14.7) (end 30.1 14.6) (width 0.25) (layer "B.Cu") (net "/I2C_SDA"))
 (segment (start 30.2 12.8) (end 30.5 12.8) (width 0.25) (layer "F.Cu") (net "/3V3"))
 (segment (start 30.2875 14.5975) (end 29.3 14.6) (width 0.2) (layer "F.Cu") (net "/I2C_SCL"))
 (segment (start 30.2875 15.0975) (end 29.3 15.1) (width 0.2) (layer "F.Cu") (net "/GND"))
 (segment (start 30.4 15.1) (end 29.3 15.1) (width 0.2) (layer "F.Cu") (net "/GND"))
 (segment (start 30.5 12.8) (end 30.5 13.4) (width 0.25) (layer "F.Cu") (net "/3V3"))
 (segment (start 30.5 13.4) (end 32.7 13.4) (width 0.25) (layer "B.Cu") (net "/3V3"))
 (segment (start 31.1 12.8) (end 31.1 15.1) (width 0.25) (layer "F.Cu") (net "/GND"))
 (segment (start 31.1 15.1) (end 30.4 15.1) (width 0.25) (layer "F.Cu") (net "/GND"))
 (segment (start 31.1 15.6) (end 31.1 15.1) (width 0.25) (layer "F.Cu") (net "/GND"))
 (segment (start 31.6 15.6) (end 31.1 15.6) (width 0.25) (layer "F.Cu") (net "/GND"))
 (segment (start 31.7 14.3) (end 31.7 14.5) (width 0.25) (layer "F.Cu") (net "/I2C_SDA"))
 (segment (start 31.7 14.5) (end 31.7 14.6) (width 0.2) (layer "F.Cu") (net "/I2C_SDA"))
 (segment (start 31.7 14.6) (end 31.7 14.3) (width 0.25) (layer "B.Cu") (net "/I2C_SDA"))
 (segment (start 31.7 14.6) (end 32.7 14.6) (width 0.2) (layer "F.Cu") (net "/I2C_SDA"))
 (segment (start 31.7125 14.5975) (end 32.7 14.6) (width 0.2) (layer "F.Cu") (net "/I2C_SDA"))
 (segment (start 31.7125 15.0975) (end 32.7 15.1) (width 0.2) (layer "F.Cu") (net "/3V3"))
 (segment (start 31.7125 15.5975) (end 32.7 15.6) (width 0.2) (layer "F.Cu") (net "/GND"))
 (segment (start 31.8 12.8) (end 31.1 12.8) (width 0.25) (layer "F.Cu") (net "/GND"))
 (segment (start 32.299999 14.6) (end 31.7 14.6) (width 0.25) (layer "B.Cu") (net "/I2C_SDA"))
 (segment (start 32.299999 15.4) (end 32.299999 14.6) (width 0.25) (layer "B.Cu") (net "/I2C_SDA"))
 (segment (start 32.4 15.4) (end 32.299999 15.4) (width 0.25) (layer "B.Cu") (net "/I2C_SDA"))
 (segment (start 32.4 15.5) (end 32.4 15.4) (width 0.25) (layer "B.Cu") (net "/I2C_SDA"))
 (segment (start 32.5 15.5) (end 32.4 15.5) (width 0.25) (layer "B.Cu") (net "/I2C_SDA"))
 (segment (start 32.5 15.6) (end 32.5 15.5) (width 0.25) (layer "B.Cu") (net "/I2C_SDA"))
 (segment (start 32.6 15.6) (end 32.5 15.6) (width 0.25) (layer "B.Cu") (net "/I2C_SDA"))
 (segment (start 32.6 15.7) (end 32.6 15.6) (width 0.25) (layer "B.Cu") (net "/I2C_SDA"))
 (segment (start 32.7 13.4) (end 32.7 15.1) (width 0.25) (layer "B.Cu") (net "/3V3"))
 (segment (start 32.7 15.1) (end 32.9 15.1) (width 0.25) (layer "B.Cu") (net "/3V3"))
 (segment (start 32.7 15.6) (end 31.6 15.6) (width 0.2) (layer "F.Cu") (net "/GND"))
 (segment (start 32.799999 15.1) (end 32.7 15.1) (width 0.2) (layer "F.Cu") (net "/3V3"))
 (segment (start 32.9 14.9) (end 32.9 15.1) (width 0.25) (layer "F.Cu") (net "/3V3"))
 (segment (start 32.9 15.1) (end 32.799999 15.1) (width 0.25) (layer "F.Cu") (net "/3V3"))
 (segment (start 33 14.8) (end 33 14.9) (width 0.25) (layer "F.Cu") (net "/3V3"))
 (segment (start 33 14.9) (end 32.9 14.9) (width 0.25) (layer "F.Cu") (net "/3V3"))
 (segment (start 33.1 14.5) (end 33.1 14.8) (width 0.25) (layer "F.Cu") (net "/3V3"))
 (segment (start 33.1 14.8) (end 33 14.8) (width 0.25) (layer "F.Cu") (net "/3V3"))
 (segment (start 33.2 15.6) (end 33.2 15.7) (width 0.25) (layer "B.Cu") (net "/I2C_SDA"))
 (segment (start 33.2 15.7) (end 32.6 15.7) (width 0.25) (layer "B.Cu") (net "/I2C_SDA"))
 (segment (start 33.299999 15.5) (end 33.299999 15.6) (width 0.25) (layer "B.Cu") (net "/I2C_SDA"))
 (segment (start 33.299999 15.6) (end 33.2 15.6) (width 0.25) (layer "B.Cu") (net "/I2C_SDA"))
 (segment (start 33.6 15.5) (end 33.299999 15.5) (width 0.25) (layer "B.Cu") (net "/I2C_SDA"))
 (segment (start 37.4 12.8) (end 31.8 12.8) (width 0.25) (layer "F.Cu") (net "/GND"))
 (segment (start 37.4 13.1) (end 37.4 12.8) (width 0.25) (layer "F.Cu") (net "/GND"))
 (segment (start 4 15) (end 5.3 15) (width 0.25) (layer "B.Cu") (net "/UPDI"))
 (segment (start 42.5 13.1) (end 37.4 13.1) (width 0.25) (layer "F.Cu") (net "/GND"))
 (segment (start 42.5 13.5) (end 42.5 13.1) (width 0.25) (layer "F.Cu") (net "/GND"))
 (segment (start 42.5 14.5) (end 33.1 14.5) (width 0.25) (layer "F.Cu") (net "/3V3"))
 (segment (start 42.5 15.5) (end 33.6 15.5) (width 0.25) (layer "F.Cu") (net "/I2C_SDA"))
 (segment (start 42.5 16.1) (end 29.7 16.1) (width 0.25) (layer "F.Cu") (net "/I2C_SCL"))
 (segment (start 42.5 16.5) (end 42.5 16.1) (width 0.25) (layer "F.Cu") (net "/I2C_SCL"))
 (segment (start 5.3 15) (end 5.3 16.2) (width 0.25) (layer "B.Cu") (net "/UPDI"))
 (segment (start 5.3 16.2) (end 14.3 16.2) (width 0.25) (layer "B.Cu") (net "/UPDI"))
 (segment (start 6.5 13.2) (end 15.3 13.2) (width 0.25) (layer "F.Cu") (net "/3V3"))
 (segment (start 6.5 15) (end 6.5 13.2) (width 0.25) (layer "F.Cu") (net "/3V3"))
 (segment (start 9.1 15) (end 16.6 15) (width 0.25) (layer "F.Cu") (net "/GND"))
 (via (at 14.7 14) (size 0.6) (drill 0.3) (layers "F.Cu" "B.Cu") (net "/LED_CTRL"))
 (via (at 15.3 16.5) (size 0.6) (drill 0.3) (layers "F.Cu" "B.Cu") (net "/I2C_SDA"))
 (via (at 16 13.6) (size 0.6) (drill 0.3) (layers "F.Cu" "B.Cu") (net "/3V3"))
 (via (at 16.9 18.1) (size 0.6) (drill 0.3) (layers "F.Cu" "B.Cu") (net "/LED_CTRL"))
 (via (at 19.1 15.7) (size 0.6) (drill 0.3) (layers "F.Cu" "B.Cu") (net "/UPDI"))
 (via (at 19.4 11) (size 0.6) (drill 0.3) (layers "F.Cu" "B.Cu") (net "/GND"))
 (via (at 21.9 14.2) (size 0.6) (drill 0.3) (layers "F.Cu" "B.Cu") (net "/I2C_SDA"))
 (via (at 24.5 15.1) (size 0.6) (drill 0.3) (layers "F.Cu" "B.Cu") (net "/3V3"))
 (via (at 28.3 14.2) (size 0.6) (drill 0.3) (layers "F.Cu" "B.Cu") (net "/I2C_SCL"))
 (via (at 29.5 14.4) (size 0.6) (drill 0.3) (layers "F.Cu" "B.Cu") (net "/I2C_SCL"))
 (via (at 30.5 13.4) (size 0.6) (drill 0.3) (layers "F.Cu" "B.Cu") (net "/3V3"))
 (via (at 31.7 14.3) (size 0.6) (drill 0.3) (layers "F.Cu" "B.Cu") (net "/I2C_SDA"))
 (via (at 32.7 12.8) (size 0.6) (drill 0.3) (layers "F.Cu" "B.Cu") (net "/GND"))
 (via (at 32.9 15.1) (size 0.6) (drill 0.3) (layers "F.Cu" "B.Cu") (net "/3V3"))
 (via (at 33.6 15.5) (size 0.6) (drill 0.3) (layers "F.Cu" "B.Cu") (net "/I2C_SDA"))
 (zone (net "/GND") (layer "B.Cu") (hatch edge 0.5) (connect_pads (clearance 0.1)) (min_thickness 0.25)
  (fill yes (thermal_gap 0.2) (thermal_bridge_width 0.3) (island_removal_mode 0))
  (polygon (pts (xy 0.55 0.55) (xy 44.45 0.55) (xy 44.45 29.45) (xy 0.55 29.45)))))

